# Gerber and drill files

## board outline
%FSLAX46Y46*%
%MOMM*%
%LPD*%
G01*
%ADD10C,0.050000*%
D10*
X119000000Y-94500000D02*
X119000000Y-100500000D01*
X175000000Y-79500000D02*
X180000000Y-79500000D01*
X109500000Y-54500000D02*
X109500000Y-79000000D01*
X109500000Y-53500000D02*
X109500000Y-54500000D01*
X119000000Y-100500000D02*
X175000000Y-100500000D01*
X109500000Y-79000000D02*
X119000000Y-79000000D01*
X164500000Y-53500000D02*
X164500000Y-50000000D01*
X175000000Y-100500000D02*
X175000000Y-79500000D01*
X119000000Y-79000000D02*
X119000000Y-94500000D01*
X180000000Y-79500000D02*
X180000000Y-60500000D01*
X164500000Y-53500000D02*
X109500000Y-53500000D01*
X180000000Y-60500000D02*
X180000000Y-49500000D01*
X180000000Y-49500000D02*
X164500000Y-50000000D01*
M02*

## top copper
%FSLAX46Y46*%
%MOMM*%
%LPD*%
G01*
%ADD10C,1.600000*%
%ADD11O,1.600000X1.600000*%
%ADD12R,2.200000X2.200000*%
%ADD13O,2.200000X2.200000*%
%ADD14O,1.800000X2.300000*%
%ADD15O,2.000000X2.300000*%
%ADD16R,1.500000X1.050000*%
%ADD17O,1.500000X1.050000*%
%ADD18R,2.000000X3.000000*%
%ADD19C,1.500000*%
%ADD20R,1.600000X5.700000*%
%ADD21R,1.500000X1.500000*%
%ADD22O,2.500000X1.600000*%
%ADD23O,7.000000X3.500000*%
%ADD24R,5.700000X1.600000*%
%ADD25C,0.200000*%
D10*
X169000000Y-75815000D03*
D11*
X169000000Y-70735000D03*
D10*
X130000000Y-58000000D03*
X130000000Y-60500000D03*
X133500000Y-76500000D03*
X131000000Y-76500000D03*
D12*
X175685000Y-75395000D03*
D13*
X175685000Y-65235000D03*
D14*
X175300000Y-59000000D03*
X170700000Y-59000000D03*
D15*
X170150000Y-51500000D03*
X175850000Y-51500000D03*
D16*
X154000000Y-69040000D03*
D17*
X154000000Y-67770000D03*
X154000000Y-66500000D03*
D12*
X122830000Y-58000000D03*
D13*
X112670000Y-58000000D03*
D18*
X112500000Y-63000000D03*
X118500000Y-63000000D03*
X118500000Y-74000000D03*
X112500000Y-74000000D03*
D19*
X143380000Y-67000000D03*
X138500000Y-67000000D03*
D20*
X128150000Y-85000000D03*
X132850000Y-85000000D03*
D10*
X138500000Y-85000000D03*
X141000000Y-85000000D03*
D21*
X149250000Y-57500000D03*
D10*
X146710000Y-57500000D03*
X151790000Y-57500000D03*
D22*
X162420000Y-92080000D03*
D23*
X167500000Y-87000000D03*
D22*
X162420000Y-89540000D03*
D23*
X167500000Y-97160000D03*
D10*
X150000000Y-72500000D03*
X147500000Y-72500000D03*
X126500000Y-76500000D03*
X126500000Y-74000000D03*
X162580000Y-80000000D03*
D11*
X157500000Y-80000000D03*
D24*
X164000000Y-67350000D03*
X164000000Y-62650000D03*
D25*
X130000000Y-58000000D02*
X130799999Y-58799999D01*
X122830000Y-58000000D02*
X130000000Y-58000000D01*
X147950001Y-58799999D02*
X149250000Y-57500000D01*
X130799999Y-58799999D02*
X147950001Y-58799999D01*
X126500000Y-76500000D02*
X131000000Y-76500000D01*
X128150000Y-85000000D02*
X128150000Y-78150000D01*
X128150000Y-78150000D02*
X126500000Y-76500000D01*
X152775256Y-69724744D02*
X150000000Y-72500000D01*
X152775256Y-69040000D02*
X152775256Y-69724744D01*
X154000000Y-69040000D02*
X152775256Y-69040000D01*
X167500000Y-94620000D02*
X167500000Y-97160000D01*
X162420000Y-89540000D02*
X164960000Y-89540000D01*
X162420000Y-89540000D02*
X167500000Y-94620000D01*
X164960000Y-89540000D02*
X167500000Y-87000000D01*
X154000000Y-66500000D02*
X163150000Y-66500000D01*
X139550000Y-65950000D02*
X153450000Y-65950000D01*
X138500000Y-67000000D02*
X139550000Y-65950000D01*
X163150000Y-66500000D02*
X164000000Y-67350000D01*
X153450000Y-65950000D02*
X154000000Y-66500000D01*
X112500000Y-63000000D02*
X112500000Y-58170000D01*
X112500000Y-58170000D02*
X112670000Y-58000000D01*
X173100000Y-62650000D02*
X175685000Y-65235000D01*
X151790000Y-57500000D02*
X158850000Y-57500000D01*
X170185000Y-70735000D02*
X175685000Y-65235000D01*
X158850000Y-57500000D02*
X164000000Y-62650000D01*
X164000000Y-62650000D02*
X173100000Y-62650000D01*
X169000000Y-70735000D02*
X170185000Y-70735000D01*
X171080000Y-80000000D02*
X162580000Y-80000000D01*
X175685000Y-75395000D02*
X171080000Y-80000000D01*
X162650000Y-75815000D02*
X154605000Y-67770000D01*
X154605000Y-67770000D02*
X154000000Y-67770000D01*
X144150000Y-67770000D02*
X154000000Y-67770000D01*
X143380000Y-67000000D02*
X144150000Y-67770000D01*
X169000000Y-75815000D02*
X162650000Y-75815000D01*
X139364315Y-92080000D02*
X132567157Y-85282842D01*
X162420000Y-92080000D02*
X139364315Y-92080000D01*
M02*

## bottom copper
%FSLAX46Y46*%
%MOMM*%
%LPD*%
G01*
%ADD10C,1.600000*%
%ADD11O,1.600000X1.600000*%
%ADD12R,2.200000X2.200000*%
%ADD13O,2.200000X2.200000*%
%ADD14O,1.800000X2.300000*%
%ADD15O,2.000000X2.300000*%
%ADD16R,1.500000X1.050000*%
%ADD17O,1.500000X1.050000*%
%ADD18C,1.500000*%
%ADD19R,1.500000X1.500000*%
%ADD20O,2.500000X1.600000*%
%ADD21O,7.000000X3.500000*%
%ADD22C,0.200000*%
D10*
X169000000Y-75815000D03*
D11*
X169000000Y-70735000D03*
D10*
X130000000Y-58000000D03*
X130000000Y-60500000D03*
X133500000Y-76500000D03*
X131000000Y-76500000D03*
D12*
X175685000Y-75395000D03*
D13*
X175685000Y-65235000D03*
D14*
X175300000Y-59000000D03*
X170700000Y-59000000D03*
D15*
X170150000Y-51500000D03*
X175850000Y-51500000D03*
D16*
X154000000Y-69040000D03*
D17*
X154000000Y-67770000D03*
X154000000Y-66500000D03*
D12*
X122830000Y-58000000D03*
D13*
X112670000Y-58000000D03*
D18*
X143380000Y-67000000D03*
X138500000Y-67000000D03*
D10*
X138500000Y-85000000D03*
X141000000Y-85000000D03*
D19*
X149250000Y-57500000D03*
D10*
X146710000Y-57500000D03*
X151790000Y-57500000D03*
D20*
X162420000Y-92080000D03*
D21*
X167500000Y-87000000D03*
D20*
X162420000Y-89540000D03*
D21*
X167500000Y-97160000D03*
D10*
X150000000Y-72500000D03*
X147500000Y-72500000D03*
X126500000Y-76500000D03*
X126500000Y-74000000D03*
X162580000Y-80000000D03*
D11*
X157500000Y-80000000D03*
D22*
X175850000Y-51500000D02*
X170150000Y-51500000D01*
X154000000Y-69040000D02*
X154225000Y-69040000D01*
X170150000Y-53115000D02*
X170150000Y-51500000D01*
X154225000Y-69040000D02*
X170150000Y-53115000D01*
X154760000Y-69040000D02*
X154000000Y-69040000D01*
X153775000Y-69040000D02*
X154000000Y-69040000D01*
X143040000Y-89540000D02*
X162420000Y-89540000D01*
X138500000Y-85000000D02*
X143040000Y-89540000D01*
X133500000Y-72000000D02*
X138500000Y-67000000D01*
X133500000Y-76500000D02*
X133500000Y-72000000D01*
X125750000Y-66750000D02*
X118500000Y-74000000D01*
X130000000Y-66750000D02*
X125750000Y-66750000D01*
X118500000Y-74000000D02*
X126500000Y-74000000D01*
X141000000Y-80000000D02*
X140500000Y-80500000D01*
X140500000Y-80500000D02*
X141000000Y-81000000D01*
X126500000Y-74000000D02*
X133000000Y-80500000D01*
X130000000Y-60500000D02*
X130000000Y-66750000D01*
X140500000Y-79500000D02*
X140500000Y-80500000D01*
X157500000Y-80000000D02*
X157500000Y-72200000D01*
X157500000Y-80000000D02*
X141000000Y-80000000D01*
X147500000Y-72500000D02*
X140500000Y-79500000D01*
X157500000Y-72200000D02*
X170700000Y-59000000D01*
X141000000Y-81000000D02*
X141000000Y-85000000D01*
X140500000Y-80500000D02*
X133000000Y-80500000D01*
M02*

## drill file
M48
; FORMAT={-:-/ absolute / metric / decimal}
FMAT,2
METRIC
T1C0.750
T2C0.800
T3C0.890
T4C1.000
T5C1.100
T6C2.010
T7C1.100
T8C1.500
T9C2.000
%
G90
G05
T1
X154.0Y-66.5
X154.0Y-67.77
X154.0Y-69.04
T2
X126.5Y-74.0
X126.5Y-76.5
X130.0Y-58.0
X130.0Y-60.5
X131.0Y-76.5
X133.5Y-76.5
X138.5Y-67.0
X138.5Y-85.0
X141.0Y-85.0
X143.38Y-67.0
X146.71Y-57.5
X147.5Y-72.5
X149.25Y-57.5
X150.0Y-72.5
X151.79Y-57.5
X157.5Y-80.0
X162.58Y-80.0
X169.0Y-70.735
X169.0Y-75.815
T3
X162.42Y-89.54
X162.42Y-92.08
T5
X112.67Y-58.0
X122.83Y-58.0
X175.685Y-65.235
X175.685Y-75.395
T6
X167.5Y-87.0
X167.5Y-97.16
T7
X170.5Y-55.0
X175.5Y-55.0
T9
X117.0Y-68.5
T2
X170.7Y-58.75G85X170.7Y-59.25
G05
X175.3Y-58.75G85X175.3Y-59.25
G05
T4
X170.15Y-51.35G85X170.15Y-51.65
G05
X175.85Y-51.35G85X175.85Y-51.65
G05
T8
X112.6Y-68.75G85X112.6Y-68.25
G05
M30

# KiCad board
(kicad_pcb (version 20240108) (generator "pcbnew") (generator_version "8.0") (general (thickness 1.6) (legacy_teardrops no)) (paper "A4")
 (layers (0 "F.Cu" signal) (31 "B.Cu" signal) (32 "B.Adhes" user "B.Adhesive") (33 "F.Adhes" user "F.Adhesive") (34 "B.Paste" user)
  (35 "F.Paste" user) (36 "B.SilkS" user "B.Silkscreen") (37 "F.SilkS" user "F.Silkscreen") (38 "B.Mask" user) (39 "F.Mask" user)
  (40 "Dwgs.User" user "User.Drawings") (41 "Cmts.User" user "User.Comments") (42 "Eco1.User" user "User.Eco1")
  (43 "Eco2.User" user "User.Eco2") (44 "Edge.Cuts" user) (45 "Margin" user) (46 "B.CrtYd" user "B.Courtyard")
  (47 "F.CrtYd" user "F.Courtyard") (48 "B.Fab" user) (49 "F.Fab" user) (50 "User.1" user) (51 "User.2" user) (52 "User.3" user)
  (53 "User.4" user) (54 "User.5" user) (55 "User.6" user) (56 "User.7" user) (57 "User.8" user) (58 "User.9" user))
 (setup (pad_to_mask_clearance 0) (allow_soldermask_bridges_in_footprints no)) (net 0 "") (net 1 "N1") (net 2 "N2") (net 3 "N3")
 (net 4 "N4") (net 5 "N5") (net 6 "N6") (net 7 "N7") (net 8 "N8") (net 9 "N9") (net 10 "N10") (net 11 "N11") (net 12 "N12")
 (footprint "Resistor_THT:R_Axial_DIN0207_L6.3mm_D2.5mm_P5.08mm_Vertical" (layer "F.Cu") (at 169 75.815 90)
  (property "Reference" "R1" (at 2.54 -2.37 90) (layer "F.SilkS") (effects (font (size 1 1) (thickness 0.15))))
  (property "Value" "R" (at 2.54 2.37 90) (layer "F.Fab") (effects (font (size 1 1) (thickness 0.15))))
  (pad "1" thru_hole circle (at 0 0 90) (size 1.6 1.6) (drill 0.8) (layers "*.Cu" "*.Mask") (remove_unused_layers no) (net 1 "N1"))
  (pad "2" thru_hole oval (at 5.08 0 90) (size 1.6 1.6) (drill 0.8) (layers "*.Cu" "*.Mask") (remove_unused_layers no) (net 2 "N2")))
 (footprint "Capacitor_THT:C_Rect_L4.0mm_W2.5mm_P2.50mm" (layer "F.Cu") (at 130 58 -90)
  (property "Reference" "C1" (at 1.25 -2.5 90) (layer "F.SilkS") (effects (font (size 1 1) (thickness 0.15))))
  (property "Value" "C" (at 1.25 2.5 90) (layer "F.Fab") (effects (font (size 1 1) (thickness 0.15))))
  (pad "1" thru_hole circle (at 0 0 270) (size 1.6 1.6) (drill 0.8) (layers "*.Cu" "*.Mask") (remove_unused_layers no) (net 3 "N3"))
  (pad "2" thru_hole circle (at 2.5 0 270) (size 1.6 1.6) (drill 0.8) (layers "*.Cu" "*.Mask") (remove_unused_layers no) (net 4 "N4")))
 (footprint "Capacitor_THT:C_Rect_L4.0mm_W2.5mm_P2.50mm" (layer "F.Cu") (at 133.5 76.5 180)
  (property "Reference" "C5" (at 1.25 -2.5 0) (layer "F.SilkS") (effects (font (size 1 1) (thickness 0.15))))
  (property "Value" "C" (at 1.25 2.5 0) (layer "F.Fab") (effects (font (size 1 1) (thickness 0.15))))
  (pad "1" thru_hole circle (at 0 0 180) (size 1.6 1.6) (drill 0.8) (layers "*.Cu" "*.Mask") (remove_unused_layers no) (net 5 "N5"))
  (pad "2" thru_hole circle (at 2.5 0 180) (size 1.6 1.6) (drill 0.8) (layers "*.Cu" "*.Mask") (remove_unused_layers no) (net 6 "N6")))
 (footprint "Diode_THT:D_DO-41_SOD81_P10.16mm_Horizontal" (layer "F.Cu") (at 175.685 75.395 90)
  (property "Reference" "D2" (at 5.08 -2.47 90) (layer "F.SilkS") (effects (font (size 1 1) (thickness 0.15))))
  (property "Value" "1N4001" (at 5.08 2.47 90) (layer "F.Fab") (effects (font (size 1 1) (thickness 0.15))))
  (pad "1" thru_hole rect (at 0 0 90) (size 2.2 2.2) (drill 1.1) (layers "*.Cu" "*.Mask") (remove_unused_layers no) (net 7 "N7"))
  (pad "2" thru_hole oval (at 10.16 0 90) (size 2.2 2.2) (drill 1.1) (layers "*.Cu" "*.Mask") (remove_unused_layers no) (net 2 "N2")))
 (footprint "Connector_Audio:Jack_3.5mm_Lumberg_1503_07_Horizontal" (layer "F.Cu") (at 170.15 51.5)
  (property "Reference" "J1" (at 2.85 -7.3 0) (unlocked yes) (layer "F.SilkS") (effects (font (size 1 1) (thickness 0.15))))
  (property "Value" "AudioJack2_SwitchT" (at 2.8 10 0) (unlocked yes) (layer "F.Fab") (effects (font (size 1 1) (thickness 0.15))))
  (pad "" np_thru_hole circle (at 0.35 3.5) (size 1.1 1.1) (drill 1.1) (layers "F&B.Cu" "*.Mask"))
  (pad "" np_thru_hole circle (at 5.35 3.5) (size 1.1 1.1) (drill 1.1) (layers "F&B.Cu" "*.Mask"))
  (pad "R" thru_hole oval (at 5.15 7.5) (size 1.8 2.3) (drill oval 0.8 1.3) (layers "*.Cu" "*.Mask") (remove_unused_layers no))
  (pad "S" thru_hole oval (at 0.55 7.5) (size 1.8 2.3) (drill oval 0.8 1.3) (layers "*.Cu" "*.Mask") (remove_unused_layers no) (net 4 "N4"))
  (pad "T" thru_hole oval (at 0 0) (size 2 2.3) (drill oval 1 1.3) (layers "*.Cu" "*.Mask") (remove_unused_layers no) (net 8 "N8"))
  (pad "T" thru_hole oval (at 5.7 0) (size 2 2.3) (drill oval 1 1.3) (layers "*.Cu" "*.Mask") (remove_unused_layers no) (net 8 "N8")))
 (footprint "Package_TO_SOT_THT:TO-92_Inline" (layer "F.Cu") (at 154 69.04 90)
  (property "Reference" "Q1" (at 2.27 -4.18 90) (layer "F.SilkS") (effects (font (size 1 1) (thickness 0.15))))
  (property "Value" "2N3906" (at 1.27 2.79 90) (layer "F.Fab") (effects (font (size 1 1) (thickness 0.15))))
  (pad "1" thru_hole rect (at 0 0 90) (size 1.05 1.5) (drill 0.75) (layers "*.Cu" "*.Mask") (remove_unused_layers no) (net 8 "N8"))
  (pad "2" thru_hole oval (at 1.27 0 90) (size 1.05 1.5) (drill 0.75) (layers "*.Cu" "*.Mask") (remove_unused_layers no) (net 1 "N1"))
  (pad "3" thru_hole oval (at 2.54 0 90) (size 1.05 1.5) (drill 0.75) (layers "*.Cu" "*.Mask") (remove_unused_layers no) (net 5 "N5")))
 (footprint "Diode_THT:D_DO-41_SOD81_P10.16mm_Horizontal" (layer "F.Cu") (at 122.83 58 180)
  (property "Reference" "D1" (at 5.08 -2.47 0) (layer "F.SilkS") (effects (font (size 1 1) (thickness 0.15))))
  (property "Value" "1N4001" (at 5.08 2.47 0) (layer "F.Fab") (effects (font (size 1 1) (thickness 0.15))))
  (pad "1" thru_hole rect (at 0 0 180) (size 2.2 2.2) (drill 1.1) (layers "*.Cu" "*.Mask") (remove_unused_layers no) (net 3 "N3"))
  (pad "2" thru_hole oval (at 10.16 0 180) (size 2.2 2.2) (drill 1.1) (layers "*.Cu" "*.Mask") (remove_unused_layers no) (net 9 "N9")))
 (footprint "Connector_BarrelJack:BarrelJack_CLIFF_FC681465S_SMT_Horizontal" (layer "F.Cu") (at 115.5 68.5)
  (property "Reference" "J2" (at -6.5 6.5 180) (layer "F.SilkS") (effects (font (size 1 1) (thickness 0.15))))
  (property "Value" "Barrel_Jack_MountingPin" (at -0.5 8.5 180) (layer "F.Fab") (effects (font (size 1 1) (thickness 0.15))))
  (pad "" np_thru_hole oval (at -2.9 0 90) (size 2 1.5) (drill oval 2 1.5) (layers "*.Cu" "*.Mask"))
  (pad "" np_thru_hole circle (at 1.5 0 90) (size 2 2) (drill 2) (layers "*.Cu" "*.Mask"))
  (pad "1" smd rect (at -3 -5.5 90) (size 3 2) (layers "F.Cu" "F.Paste" "F.Mask") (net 9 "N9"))
  (pad "1" smd rect (at 3 -5.5 90) (size 3 2) (layers "F.Cu" "F.Paste" "F.Mask") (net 9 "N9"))
  (pad "2" smd rect (at 3 5.5 90) (size 3 2) (layers "F.Cu" "F.Paste" "F.Mask") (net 4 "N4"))
  (pad "3" smd rect (at -3 5.5 90) (size 3 2) (layers "F.Cu" "F.Paste" "F.Mask")))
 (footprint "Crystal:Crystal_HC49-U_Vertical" (layer "F.Cu") (at 143.38 67 180)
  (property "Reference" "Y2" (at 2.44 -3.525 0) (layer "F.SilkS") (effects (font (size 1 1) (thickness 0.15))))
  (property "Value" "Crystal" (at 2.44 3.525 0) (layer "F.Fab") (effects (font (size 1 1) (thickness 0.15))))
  (pad "1" thru_hole circle (at 0 0 180) (size 1.5 1.5) (drill 0.8) (layers "*.Cu" "*.Mask") (remove_unused_layers no) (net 1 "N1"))
  (pad "2" thru_hole circle (at 4.88 0 180) (size 1.5 1.5) (drill 0.8) (layers "*.Cu" "*.Mask") (remove_unused_layers no) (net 5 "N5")))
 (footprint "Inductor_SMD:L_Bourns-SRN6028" (layer "F.Cu") (at 130.5 85)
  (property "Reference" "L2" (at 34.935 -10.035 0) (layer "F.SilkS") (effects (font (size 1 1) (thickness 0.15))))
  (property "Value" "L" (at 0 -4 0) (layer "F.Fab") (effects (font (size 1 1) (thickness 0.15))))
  (pad "1" smd rect (at -2.35 0) (size 1.6 5.7) (layers "F.Cu" "F.Paste" "F.Mask") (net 6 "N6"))
  (pad "2" smd rect (at 2.35 0) (size 1.6 5.7) (layers "F.Cu" "F.Paste" "F.Mask") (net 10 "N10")))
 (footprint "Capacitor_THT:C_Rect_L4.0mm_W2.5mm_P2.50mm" (layer "F.Cu") (at 138.5 85)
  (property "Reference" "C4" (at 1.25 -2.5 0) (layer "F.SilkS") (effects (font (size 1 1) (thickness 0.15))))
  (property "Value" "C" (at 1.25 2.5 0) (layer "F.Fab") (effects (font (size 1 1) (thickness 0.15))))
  (pad "1" thru_hole circle (at 0 0) (size 1.6 1.6) (drill 0.8) (layers "*.Cu" "*.Mask") (remove_unused_layers no) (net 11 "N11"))
  (pad "2" thru_hole circle (at 2.5 0) (size 1.6 1.6) (drill 0.8) (layers "*.Cu" "*.Mask") (remove_unused_layers no) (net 4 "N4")))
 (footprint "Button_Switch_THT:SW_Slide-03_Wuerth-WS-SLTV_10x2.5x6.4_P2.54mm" (layer "F.Cu") (at 149.25 57.5)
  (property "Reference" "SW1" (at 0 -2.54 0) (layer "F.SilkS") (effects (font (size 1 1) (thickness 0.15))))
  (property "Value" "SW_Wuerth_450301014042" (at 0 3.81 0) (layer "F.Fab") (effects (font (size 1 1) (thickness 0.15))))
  (pad "1" thru_hole rect (at 0 0) (size 1.5 1.5) (drill 0.8) (layers "*.Cu" "*.Mask") (remove_unused_layers no) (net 3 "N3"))
  (pad "2" thru_hole circle (at -2.54 0) (size 1.6 1.6) (drill 0.8) (layers "*.Cu" "*.Mask") (remove_unused_layers no) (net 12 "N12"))
  (pad "3" thru_hole circle (at 2.54 0) (size 1.6 1.6) (drill 0.8) (layers "*.Cu" "*.Mask") (remove_unused_layers no) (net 2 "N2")))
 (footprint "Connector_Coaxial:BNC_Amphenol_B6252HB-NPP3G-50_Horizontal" (layer "F.Cu") (at 162.42 92.08 -90)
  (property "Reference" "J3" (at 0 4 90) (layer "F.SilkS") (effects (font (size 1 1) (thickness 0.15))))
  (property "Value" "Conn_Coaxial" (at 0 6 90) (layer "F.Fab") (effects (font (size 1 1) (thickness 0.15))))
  (pad "1" thru_hole oval (at 0 0 270) (size 1.6 2.5) (drill 0.89) (layers "*.Cu" "*.Mask") (remove_unused_layers no) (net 10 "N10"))
  (pad "2" thru_hole oval (at -5.08 -5.08 270) (size 3.5 7) (drill 2.01) (layers "*.Cu" "*.Mask") (remove_unused_layers no) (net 11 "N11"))
  (pad "2" thru_hole oval (at -2.54 0 270) (size 1.6 2.5) (drill 0.89) (layers "*.Cu" "*.Mask") (remove_unused_layers no) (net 11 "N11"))
  (pad "2" thru_hole oval (at 5.08 -5.08 270) (size 3.5 7) (drill 2.01) (layers "*.Cu" "*.Mask") (remove_unused_layers no) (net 11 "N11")))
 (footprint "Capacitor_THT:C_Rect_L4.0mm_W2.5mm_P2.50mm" (layer "F.Cu") (at 150 72.5 180)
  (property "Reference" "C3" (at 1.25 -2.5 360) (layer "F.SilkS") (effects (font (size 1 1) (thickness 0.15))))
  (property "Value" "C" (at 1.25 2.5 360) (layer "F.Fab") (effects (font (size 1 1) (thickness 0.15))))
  (pad "1" thru_hole circle (at 0 0 180) (size 1.6 1.6) (drill 0.8) (layers "*.Cu" "*.Mask") (remove_unused_layers no) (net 8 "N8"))
  (pad "2" thru_hole circle (at 2.5 0 180) (size 1.6 1.6) (drill 0.8) (layers "*.Cu" "*.Mask") (remove_unused_layers no) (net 4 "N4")))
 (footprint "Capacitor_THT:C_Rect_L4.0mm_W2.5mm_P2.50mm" (layer "F.Cu") (at 126.5 76.5 90)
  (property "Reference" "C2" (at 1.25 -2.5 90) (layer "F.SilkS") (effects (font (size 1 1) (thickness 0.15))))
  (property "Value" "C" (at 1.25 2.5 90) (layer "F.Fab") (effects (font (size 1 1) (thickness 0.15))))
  (pad "1" thru_hole circle (at 0 0 90) (size 1.6 1.6) (drill 0.8) (layers "*.Cu" "*.Mask") (remove_unused_layers no) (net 6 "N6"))
  (pad "2" thru_hole circle (at 2.5 0 90) (size 1.6 1.6) (drill 0.8) (layers "*.Cu" "*.Mask") (remove_unused_layers no) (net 4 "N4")))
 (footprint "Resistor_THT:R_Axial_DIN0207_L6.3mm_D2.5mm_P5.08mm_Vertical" (layer "F.Cu") (at 162.58 80 180)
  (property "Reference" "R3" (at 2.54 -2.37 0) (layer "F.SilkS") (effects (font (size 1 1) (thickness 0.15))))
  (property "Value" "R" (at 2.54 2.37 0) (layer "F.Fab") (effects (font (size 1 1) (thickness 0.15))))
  (pad "1" thru_hole circle (at 0 0 180) (size 1.6 1.6) (drill 0.8) (layers "*.Cu" "*.Mask") (remove_unused_layers no) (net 7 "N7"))
  (pad "2" thru_hole oval (at 5.08 0 180) (size 1.6 1.6) (drill 0.8) (layers "*.Cu" "*.Mask") (remove_unused_layers no) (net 4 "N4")))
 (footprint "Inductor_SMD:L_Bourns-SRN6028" (layer "F.Cu") (at 164 65 90)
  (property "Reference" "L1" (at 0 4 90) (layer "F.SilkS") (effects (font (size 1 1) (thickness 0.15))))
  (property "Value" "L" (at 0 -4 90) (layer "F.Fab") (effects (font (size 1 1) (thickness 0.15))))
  (pad "1" smd rect (at -2.35 0 90) (size 1.6 5.7) (layers "F.Cu" "F.Paste" "F.Mask") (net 5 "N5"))
  (pad "2" smd rect (at 2.35 0 90) (size 1.6 5.7) (layers "F.Cu" "F.Paste" "F.Mask") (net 2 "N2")))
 (gr_line (start 119 94.5) (end 119 100.5) (stroke (width 0.05) (type default)) (layer "Edge.Cuts"))
 (gr_line (start 175 79.5) (end 180 79.5) (stroke (width 0.05) (type default)) (layer "Edge.Cuts"))
 (gr_line (start 109.5 54.5) (end 109.5 79) (stroke (width 0.05) (type default)) (layer "Edge.Cuts"))
 (gr_line (start 109.5 53.5) (end 109.5 54.5) (stroke (width 0.05) (type default)) (layer "Edge.Cuts"))
 (gr_line (start 119 100.5) (end 175 100.5) (stroke (width 0.05) (type default)) (layer "Edge.Cuts"))
 (gr_line (start 109.5 79) (end 119 79) (stroke (width 0.05) (type default)) (layer "Edge.Cuts"))
 (gr_line (start 164.5 53.5) (end 164.5 50) (stroke (width 0.05) (type default)) (layer "Edge.Cuts"))
 (gr_line (start 175 100.5) (end 175 79.5) (stroke (width 0.05) (type default)) (layer "Edge.Cuts"))
 (gr_line (start 119 79) (end 119 94.5) (stroke (width 0.05) (type default)) (layer "Edge.Cuts"))
 (gr_line (start 180 79.5) (end 180 60.5) (stroke (width 0.05) (type default)) (layer "Edge.Cuts"))
 (gr_line (start 164.5 53.5) (end 109.5 53.5) (stroke (width 0.05) (type default)) (layer "Edge.Cuts"))
 (gr_line (start 180 60.5) (end 180 49.5) (stroke (width 0.05) (type default)) (layer "Edge.Cuts"))
 (gr_line (start 180 49.5) (end 164.5 50) (stroke (width 0.05) (type default)) (layer "Edge.Cuts"))
 (segment (start 130 58) (end 130.799999 58.799999) (width 0.2) (layer "F.Cu") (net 3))
 (segment (start 122.83 58) (end 130 58) (width 0.2) (layer "F.Cu") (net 3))
 (segment (start 147.950001 58.799999) (end 149.25 57.5) (width 0.2) (layer "F.Cu") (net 3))
 (segment (start 130.799999 58.799999) (end 147.950001 58.799999) (width 0.2) (layer "F.Cu") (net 3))
 (segment (start 126.5 76.5) (end 131 76.5) (width 0.2) (layer "F.Cu") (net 6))
 (segment (start 128.15 85) (end 128.15 78.15) (width 0.2) (layer "F.Cu") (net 6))
 (segment (start 128.15 78.15) (end 126.5 76.5) (width 0.2) (layer "F.Cu") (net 6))
 (segment (start 152.775256 69.724744) (end 150 72.5) (width 0.2) (layer "F.Cu") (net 8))
 (segment (start 152.775256 69.04) (end 152.775256 69.724744) (width 0.2) (layer "F.Cu") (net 8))
 (segment (start 154 69.04) (end 152.775256 69.04) (width 0.2) (layer "F.Cu") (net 8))
 (segment (start 175.85 51.5) (end 170.15 51.5) (width 0.2) (layer "B.Cu") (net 8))
 (segment (start 154 69.04) (end 154.225 69.04) (width 0.2) (layer "B.Cu") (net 8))
 (segment (start 170.15 53.115) (end 170.15 51.5) (width 0.2) (layer "B.Cu") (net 8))
 (segment (start 154.225 69.04) (end 170.15 53.115) (width 0.2) (layer "B.Cu") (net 8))
 (segment (start 154.76 69.04) (end 154 69.04) (width 0.2) (layer "B.Cu") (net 8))
 (segment (start 153.775 69.04) (end 154 69.04) (width 0.2) (layer "B.Cu") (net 8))
 (segment (start 167.5 94.62) (end 167.5 97.16) (width 0.2) (layer "F.Cu") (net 11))
 (segment (start 162.42 89.54) (end 164.96 89.54) (width 0.2) (layer "F.Cu") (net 11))
 (segment (start 162.42 89.54) (end 167.5 94.62) (width 0.2) (layer "F.Cu") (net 11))
 (segment (start 164.96 89.54) (end 167.5 87) (width 0.2) (layer "F.Cu") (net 11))
 (segment (start 143.04 89.54) (end 162.42 89.54) (width 0.2) (layer "B.Cu") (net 11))
 (segment (start 138.5 85) (end 143.04 89.54) (width 0.2) (layer "B.Cu") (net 11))
 (segment (start 154 66.5) (end 163.15 66.5) (width 0.2) (layer "F.Cu") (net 5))
 (segment (start 139.55 65.95) (end 153.45 65.95) (width 0.2) (layer "F.Cu") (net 5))
 (segment (start 138.5 67) (end 139.55 65.95) (width 0.2) (layer "F.Cu") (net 5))
 (segment (start 163.15 66.5) (end 164 67.35) (width 0.2) (layer "F.Cu") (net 5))
 (segment (start 153.45 65.95) (end 154 66.5) (width 0.2) (layer "F.Cu") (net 5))
 (segment (start 133.5 72) (end 138.5 67) (width 0.2) (layer "B.Cu") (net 5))
 (segment (start 133.5 76.5) (end 133.5 72) (width 0.2) (layer "B.Cu") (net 5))
 (segment (start 112.5 63) (end 112.5 58.17) (width 0.2) (layer "F.Cu") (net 9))
 (segment (start 112.5 58.17) (end 112.67 58) (width 0.2) (layer "F.Cu") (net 9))
 (segment (start 173.1 62.65) (end 175.685 65.235) (width 0.2) (layer "F.Cu") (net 2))
 (segment (start 151.79 57.5) (end 158.85 57.5) (width 0.2) (layer "F.Cu") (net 2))
 (segment (start 170.185 70.735) (end 175.685 65.235) (width 0.2) (layer "F.Cu") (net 2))
 (segment (start 158.85 57.5) (end 164 62.65) (width 0.2) (layer "F.Cu") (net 2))
 (segment (start 164 62.65) (end 173.1 62.65) (width 0.2) (layer "F.Cu") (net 2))
 (segment (start 169 70.735) (end 170.185 70.735) (width 0.2) (layer "F.Cu") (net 2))
 (segment (start 171.08 80) (end 162.58 80) (width 0.2) (layer "F.Cu") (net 7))
 (segment (start 175.685 75.395) (end 171.08 80) (width 0.2) (layer "F.Cu") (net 7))
 (segment (start 162.65 75.815) (end 154.605 67.77) (width 0.2) (layer "F.Cu") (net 1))
 (segment (start 154.605 67.77) (end 154 67.77) (width 0.2) (layer "F.Cu") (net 1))
 (segment (start 144.15 67.77) (end 154 67.77) (width 0.2) (layer "F.Cu") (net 1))
 (segment (start 143.38 67) (end 144.15 67.77) (width 0.2) (layer "F.Cu") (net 1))
 (segment (start 169 75.815) (end 162.65 75.815) (width 0.2) (layer "F.Cu") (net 1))
 (segment (start 139.364315 92.08) (end 132.567157 85.282842) (width 0.2) (layer "F.Cu") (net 10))
 (segment (start 162.42 92.08) (end 139.364315 92.08) (width 0.2) (layer "F.Cu") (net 10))
 (segment (start 125.75 66.75) (end 118.5 74) (width 0.2) (layer "B.Cu") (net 4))
 (segment (start 130 66.75) (end 125.75 66.75) (width 0.2) (layer "B.Cu") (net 4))
 (segment (start 118.5 74) (end 126.5 74) (width 0.2) (layer "B.Cu") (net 4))
 (segment (start 141 80) (end 140.5 80.5) (width 0.2) (layer "B.Cu") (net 4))
 (segment (start 140.5 80.5) (end 141 81) (width 0.2) (layer "B.Cu") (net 4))
 (segment (start 126.5 74) (end 133 80.5) (width 0.2) (layer "B.Cu") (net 4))
 (segment (start 130 60.5) (end 130 66.75) (width 0.2) (layer "B.Cu") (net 4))
 (segment (start 140.5 79.5) (end 140.5 80.5) (width 0.2) (layer "B.Cu") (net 4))
 (segment (start 157.5 80) (end 157.5 72.2) (width 0.2) (layer "B.Cu") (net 4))
 (segment (start 157.5 80) (end 141 80) (width 0.2) (layer "B.Cu") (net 4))
 (segment (start 147.5 72.5) (end 140.5 79.5) (width 0.2) (layer "B.Cu") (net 4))
 (segment (start 157.5 72.2) (end 170.7 59) (width 0.2) (layer "B.Cu") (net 4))
 (segment (start 141 81) (end 141 85) (width 0.2) (layer "B.Cu") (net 4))
 (segment (start 140.5 80.5) (end 133 80.5) (width 0.2) (layer "B.Cu") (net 4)))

